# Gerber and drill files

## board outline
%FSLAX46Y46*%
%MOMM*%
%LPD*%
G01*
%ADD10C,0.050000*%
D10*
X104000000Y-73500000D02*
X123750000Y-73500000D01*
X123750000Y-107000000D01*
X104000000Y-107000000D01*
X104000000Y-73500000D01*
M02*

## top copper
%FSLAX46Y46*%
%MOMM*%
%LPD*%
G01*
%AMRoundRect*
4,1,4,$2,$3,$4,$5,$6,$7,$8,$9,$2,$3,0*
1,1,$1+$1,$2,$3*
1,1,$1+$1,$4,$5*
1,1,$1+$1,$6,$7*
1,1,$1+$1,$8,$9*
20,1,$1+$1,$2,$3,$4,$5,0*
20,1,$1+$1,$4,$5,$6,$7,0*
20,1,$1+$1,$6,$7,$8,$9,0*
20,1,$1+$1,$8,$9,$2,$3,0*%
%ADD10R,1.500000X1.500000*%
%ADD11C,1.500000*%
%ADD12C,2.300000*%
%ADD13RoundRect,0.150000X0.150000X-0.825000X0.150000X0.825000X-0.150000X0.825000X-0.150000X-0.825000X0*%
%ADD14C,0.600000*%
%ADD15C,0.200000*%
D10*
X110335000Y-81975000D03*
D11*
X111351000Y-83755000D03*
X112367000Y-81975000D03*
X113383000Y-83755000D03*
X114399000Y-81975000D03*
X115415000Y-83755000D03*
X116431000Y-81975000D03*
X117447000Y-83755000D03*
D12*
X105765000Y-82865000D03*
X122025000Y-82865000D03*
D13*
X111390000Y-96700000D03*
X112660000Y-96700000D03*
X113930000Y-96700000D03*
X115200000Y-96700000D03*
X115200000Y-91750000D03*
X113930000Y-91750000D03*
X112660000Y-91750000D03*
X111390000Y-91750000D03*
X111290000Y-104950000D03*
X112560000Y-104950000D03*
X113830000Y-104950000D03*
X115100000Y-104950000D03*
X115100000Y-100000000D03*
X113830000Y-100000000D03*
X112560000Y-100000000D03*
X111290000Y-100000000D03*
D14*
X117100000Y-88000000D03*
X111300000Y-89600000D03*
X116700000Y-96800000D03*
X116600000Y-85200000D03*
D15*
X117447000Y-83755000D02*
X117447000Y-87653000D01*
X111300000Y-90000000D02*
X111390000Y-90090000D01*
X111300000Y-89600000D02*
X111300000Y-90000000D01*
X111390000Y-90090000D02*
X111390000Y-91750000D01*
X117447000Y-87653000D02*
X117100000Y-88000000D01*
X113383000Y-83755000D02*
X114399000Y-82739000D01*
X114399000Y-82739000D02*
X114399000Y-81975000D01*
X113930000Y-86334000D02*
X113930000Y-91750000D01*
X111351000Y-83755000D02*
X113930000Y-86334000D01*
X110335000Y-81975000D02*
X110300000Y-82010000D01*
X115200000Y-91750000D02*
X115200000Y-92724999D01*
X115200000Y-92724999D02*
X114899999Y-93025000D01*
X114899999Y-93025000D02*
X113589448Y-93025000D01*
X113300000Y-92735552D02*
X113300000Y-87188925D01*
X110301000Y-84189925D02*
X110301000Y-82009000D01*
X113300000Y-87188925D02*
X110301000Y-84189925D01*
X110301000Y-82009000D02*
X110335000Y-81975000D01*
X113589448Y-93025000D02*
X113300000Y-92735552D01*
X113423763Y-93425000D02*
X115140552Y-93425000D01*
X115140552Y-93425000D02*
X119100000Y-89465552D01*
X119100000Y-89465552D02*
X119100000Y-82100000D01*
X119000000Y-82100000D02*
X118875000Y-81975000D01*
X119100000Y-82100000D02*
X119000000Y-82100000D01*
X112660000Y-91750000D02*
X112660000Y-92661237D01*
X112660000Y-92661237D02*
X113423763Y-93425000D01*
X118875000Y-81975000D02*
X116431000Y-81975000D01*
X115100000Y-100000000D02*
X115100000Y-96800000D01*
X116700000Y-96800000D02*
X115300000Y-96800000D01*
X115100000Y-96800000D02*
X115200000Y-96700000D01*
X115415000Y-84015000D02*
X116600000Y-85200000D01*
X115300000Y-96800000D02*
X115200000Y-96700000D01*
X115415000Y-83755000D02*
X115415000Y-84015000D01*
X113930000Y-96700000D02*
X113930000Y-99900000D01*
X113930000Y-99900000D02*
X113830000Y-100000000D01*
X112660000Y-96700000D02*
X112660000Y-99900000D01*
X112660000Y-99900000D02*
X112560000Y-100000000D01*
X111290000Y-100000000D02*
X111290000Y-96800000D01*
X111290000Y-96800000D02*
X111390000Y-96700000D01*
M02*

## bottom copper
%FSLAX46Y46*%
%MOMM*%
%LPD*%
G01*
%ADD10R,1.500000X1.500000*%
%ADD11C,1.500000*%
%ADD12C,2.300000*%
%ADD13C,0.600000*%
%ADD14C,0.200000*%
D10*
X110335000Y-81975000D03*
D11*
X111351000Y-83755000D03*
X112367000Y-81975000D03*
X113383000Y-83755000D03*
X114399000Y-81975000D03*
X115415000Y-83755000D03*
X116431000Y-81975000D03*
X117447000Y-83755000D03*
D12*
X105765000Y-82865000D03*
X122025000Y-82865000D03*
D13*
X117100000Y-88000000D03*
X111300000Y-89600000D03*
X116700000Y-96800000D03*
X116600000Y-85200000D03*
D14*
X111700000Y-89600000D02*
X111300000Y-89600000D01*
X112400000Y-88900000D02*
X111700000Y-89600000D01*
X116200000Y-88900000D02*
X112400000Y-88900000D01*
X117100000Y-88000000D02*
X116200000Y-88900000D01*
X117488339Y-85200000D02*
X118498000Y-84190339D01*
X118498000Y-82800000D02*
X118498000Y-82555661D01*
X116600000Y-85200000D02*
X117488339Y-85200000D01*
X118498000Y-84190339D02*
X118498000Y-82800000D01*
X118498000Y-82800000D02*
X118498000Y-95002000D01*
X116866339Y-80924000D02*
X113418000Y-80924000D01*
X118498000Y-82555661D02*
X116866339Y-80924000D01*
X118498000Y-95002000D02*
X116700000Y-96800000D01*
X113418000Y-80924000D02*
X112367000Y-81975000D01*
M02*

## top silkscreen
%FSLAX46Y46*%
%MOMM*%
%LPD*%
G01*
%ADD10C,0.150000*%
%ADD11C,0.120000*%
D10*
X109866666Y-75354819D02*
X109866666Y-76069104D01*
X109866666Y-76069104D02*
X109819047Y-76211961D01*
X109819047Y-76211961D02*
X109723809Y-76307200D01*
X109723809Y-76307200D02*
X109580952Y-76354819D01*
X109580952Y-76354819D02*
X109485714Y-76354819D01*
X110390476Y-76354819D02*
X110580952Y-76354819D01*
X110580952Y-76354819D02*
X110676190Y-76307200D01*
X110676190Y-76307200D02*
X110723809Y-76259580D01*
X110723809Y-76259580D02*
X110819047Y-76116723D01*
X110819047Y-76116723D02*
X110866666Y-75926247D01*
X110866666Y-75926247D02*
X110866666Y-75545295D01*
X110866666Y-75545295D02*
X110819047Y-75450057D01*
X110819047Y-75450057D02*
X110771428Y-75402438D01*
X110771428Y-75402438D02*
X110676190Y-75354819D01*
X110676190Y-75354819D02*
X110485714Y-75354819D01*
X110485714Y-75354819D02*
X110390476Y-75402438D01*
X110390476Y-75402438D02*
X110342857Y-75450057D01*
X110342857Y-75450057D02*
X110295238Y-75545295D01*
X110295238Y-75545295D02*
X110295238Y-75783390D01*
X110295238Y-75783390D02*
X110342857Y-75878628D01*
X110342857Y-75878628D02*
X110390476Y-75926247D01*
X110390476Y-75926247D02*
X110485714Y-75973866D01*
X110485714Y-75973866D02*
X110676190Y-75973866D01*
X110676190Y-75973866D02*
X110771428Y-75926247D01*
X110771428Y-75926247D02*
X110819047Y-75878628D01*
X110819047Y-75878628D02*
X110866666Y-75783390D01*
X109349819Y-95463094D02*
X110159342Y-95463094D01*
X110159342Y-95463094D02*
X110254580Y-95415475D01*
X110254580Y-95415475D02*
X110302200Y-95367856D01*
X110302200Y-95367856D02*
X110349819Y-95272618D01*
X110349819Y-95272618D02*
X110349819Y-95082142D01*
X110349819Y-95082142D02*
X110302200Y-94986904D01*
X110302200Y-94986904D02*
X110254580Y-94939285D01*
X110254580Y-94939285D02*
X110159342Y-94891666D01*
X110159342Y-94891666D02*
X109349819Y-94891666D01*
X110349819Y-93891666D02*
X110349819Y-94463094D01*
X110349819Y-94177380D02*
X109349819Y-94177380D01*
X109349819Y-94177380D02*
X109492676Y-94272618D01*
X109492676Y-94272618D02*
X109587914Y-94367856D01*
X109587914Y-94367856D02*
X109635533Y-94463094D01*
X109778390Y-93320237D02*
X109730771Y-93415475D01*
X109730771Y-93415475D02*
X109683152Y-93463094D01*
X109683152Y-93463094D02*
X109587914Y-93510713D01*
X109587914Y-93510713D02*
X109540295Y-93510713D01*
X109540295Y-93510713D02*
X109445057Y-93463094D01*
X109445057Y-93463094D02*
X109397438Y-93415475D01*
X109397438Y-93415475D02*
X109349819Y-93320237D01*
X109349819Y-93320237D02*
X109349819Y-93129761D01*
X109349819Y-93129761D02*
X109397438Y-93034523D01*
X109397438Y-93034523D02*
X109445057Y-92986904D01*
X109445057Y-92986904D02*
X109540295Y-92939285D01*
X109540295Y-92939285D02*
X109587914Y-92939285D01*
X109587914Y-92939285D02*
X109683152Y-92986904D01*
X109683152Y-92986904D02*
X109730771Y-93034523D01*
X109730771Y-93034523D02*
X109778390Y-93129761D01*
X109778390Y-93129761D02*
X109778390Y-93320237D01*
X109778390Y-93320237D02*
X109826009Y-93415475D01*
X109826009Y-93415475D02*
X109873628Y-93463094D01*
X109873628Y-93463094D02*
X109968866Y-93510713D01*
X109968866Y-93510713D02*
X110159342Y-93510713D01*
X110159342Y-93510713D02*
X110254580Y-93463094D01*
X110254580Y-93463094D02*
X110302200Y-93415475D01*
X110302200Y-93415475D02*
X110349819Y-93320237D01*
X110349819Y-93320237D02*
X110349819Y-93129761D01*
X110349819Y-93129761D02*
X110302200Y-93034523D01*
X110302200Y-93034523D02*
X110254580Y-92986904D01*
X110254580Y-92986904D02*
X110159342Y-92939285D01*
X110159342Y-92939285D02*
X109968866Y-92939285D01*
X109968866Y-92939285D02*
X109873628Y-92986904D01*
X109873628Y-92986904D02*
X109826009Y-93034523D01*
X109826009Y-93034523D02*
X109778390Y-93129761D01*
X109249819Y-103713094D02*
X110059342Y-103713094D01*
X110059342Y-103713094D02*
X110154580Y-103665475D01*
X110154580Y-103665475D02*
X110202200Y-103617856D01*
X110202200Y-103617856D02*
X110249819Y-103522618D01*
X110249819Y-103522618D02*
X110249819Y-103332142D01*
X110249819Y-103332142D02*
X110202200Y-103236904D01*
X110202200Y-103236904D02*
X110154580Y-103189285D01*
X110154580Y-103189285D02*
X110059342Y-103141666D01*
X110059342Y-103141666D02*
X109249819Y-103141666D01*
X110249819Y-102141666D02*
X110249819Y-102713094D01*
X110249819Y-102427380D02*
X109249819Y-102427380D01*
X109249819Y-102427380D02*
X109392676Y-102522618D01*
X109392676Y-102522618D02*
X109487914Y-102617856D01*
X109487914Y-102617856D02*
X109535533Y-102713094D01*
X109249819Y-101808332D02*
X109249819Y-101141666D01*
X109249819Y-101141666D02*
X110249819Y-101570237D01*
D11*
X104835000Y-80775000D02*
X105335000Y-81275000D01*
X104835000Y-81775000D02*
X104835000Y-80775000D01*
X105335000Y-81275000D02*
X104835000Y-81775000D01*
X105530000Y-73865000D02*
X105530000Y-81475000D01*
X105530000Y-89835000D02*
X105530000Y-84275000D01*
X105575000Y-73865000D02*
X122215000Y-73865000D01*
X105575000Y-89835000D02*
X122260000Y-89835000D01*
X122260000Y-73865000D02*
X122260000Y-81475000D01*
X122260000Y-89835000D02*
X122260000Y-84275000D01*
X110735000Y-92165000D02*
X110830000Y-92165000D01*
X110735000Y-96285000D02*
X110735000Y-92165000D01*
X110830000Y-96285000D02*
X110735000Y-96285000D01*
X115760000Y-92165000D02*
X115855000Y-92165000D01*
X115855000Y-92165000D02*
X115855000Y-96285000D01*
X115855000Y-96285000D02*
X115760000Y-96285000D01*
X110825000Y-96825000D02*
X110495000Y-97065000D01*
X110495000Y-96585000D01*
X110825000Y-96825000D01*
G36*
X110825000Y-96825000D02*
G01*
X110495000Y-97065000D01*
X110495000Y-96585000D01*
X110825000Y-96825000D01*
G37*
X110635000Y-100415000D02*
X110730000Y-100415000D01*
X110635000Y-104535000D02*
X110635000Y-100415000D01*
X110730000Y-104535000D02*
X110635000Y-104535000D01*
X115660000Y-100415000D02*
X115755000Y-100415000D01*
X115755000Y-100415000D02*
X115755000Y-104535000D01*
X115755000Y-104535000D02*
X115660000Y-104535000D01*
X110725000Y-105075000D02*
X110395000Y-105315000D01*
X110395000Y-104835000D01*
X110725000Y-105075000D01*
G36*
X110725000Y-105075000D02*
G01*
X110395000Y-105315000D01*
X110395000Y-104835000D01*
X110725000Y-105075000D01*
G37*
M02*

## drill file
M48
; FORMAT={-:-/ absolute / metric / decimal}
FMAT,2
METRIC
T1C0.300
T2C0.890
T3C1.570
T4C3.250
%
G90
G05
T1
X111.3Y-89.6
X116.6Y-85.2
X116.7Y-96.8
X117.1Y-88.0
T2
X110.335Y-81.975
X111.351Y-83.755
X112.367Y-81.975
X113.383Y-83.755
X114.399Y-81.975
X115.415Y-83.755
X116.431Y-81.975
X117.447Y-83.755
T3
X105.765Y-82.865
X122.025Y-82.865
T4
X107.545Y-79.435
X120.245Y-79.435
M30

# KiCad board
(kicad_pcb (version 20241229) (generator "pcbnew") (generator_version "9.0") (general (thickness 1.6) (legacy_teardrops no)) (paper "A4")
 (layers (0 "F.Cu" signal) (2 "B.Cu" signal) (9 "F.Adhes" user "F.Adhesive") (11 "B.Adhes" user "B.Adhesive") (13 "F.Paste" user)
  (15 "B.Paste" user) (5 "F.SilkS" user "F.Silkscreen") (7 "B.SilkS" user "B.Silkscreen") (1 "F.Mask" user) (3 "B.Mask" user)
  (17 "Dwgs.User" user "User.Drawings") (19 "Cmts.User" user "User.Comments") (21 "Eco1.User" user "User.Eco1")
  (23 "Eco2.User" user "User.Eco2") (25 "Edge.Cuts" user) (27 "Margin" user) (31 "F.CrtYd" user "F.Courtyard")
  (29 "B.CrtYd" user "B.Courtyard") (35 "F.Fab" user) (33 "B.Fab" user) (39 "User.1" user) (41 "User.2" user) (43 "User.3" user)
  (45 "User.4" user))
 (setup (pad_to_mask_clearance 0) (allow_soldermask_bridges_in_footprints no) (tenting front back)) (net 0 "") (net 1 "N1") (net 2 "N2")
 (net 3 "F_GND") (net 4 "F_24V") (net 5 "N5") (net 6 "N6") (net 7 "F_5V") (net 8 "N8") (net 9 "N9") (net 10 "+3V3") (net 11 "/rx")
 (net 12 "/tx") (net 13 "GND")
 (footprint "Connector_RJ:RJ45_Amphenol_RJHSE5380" (layer "F.Cu") (at 110.335 81.975)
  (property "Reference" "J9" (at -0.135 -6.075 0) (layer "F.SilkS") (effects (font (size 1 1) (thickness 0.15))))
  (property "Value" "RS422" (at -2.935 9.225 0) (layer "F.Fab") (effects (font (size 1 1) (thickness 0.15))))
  (fp_line (start -5.5 -1.2) (end -5 -0.7) (stroke (width 0.12) (type solid)) (layer "F.SilkS"))
  (fp_line (start -5.5 -0.2) (end -5.5 -1.2) (stroke (width 0.12) (type solid)) (layer "F.SilkS"))
  (fp_line (start -5 -0.7) (end -5.5 -0.2) (stroke (width 0.12) (type solid)) (layer "F.SilkS"))
  (fp_line (start -4.805 -8.11) (end -4.805 -0.5) (stroke (width 0.12) (type solid)) (layer "F.SilkS"))
  (fp_line (start -4.805 7.86) (end -4.805 2.3) (stroke (width 0.12) (type solid)) (layer "F.SilkS"))
  (fp_line (start -4.76 -8.11) (end 11.88 -8.11) (stroke (width 0.12) (type solid)) (layer "F.SilkS"))
  (fp_line (start -4.76 7.86) (end 11.925 7.86) (stroke (width 0.12) (type solid)) (layer "F.SilkS"))
  (fp_line (start 11.925 -8.11) (end 11.925 -0.5) (stroke (width 0.12) (type solid)) (layer "F.SilkS"))
  (fp_line (start 11.925 7.86) (end 11.925 2.3) (stroke (width 0.12) (type solid)) (layer "F.SilkS"))
  (pad "" np_thru_hole circle (at -2.79 -2.54) (size 3.25 3.25) (drill 3.25) (layers "*.Cu" "*.Mask"))
  (pad "" np_thru_hole circle (at 9.91 -2.54) (size 3.25 3.25) (drill 3.25) (layers "*.Cu" "*.Mask"))
  (pad "1" thru_hole rect (at 0 0) (size 1.5 1.5) (drill 0.89) (layers "*.Cu" "*.Mask") (remove_unused_layers no) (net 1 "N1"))
  (pad "2" thru_hole circle (at 1.016 1.78) (size 1.5 1.5) (drill 0.89) (layers "*.Cu" "*.Mask") (remove_unused_layers no) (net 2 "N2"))
  (pad "3" thru_hole circle (at 2.032 0) (size 1.5 1.5) (drill 0.89) (layers "*.Cu" "*.Mask") (remove_unused_layers no) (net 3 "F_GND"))
  (pad "4" thru_hole circle (at 3.048 1.78) (size 1.5 1.5) (drill 0.89) (layers "*.Cu" "*.Mask") (remove_unused_layers no) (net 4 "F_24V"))
  (pad "5" thru_hole circle (at 4.064 0) (size 1.5 1.5) (drill 0.89) (layers "*.Cu" "*.Mask") (remove_unused_layers no) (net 4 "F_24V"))
  (pad "6" thru_hole circle (at 5.08 1.78) (size 1.5 1.5) (drill 0.89) (layers "*.Cu" "*.Mask") (remove_unused_layers no) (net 3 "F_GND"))
  (pad "7" thru_hole circle (at 6.096 0) (size 1.5 1.5) (drill 0.89) (layers "*.Cu" "*.Mask") (remove_unused_layers no) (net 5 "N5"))
  (pad "8" thru_hole circle (at 7.112 1.78) (size 1.5 1.5) (drill 0.89) (layers "*.Cu" "*.Mask") (remove_unused_layers no) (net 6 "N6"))
  (pad "SH" thru_hole circle (at -4.57 0.89) (size 2.3 2.3) (drill 1.57) (layers "*.Cu" "*.Mask") (remove_unused_layers no))
  (pad "SH" thru_hole circle (at 11.69 0.89) (size 2.3 2.3) (drill 1.57) (layers "*.Cu" "*.Mask") (remove_unused_layers no)))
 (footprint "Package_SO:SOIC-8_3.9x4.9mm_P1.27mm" (layer "F.Cu") (at 113.295 94.225 90)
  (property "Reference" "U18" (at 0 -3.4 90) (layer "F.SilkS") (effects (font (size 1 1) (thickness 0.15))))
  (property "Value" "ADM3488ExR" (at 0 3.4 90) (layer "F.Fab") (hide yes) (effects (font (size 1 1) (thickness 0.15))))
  (fp_line (start 2.06 -2.56) (end 2.06 -2.465) (stroke (width 0.12) (type solid)) (layer "F.SilkS"))
  (fp_line (start -2.06 -2.56) (end 2.06 -2.56) (stroke (width 0.12) (type solid)) (layer "F.SilkS"))
  (fp_line (start -2.06 -2.465) (end -2.06 -2.56) (stroke (width 0.12) (type solid)) (layer "F.SilkS"))
  (fp_line (start 2.06 2.465) (end 2.06 2.56) (stroke (width 0.12) (type solid)) (layer "F.SilkS"))
  (fp_line (start 2.06 2.56) (end -2.06 2.56) (stroke (width 0.12) (type solid)) (layer "F.SilkS"))
  (fp_line (start -2.06 2.56) (end -2.06 2.465) (stroke (width 0.12) (type solid)) (layer "F.SilkS"))
  (fp_poly (pts (xy -2.6 -2.47) (xy -2.84 -2.8) (xy -2.36 -2.8)) (stroke (width 0.12) (type solid)) (fill yes) (layer "F.SilkS"))
  (pad "1" smd roundrect (at -2.475 -1.905 90) (size 1.95 0.6) (layers "F.Cu" "F.Mask" "F.Paste") (roundrect_rratio 0.25) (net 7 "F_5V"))
  (pad "2" smd roundrect (at -2.475 -0.635 90) (size 1.95 0.6) (layers "F.Cu" "F.Mask" "F.Paste") (roundrect_rratio 0.25) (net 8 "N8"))
  (pad "3" smd roundrect (at -2.475 0.635 90) (size 1.95 0.6) (layers "F.Cu" "F.Mask" "F.Paste") (roundrect_rratio 0.25) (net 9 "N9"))
  (pad "4" smd roundrect (at -2.475 1.905 90) (size 1.95 0.6) (layers "F.Cu" "F.Mask" "F.Paste") (roundrect_rratio 0.25) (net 3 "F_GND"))
  (pad "5" smd roundrect (at 2.475 1.905 90) (size 1.95 0.6) (layers "F.Cu" "F.Mask" "F.Paste") (roundrect_rratio 0.25) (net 1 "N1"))
  (pad "6" smd roundrect (at 2.475 0.635 90) (size 1.95 0.6) (layers "F.Cu" "F.Mask" "F.Paste") (roundrect_rratio 0.25) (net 2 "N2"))
  (pad "7" smd roundrect (at 2.475 -0.635 90) (size 1.95 0.6) (layers "F.Cu" "F.Mask" "F.Paste") (roundrect_rratio 0.25) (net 5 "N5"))
  (pad "8" smd roundrect (at 2.475 -1.905 90) (size 1.95 0.6) (layers "F.Cu" "F.Mask" "F.Paste") (roundrect_rratio 0.25) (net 6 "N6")))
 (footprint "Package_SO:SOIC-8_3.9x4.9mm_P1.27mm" (layer "F.Cu") (at 113.195 102.475 90)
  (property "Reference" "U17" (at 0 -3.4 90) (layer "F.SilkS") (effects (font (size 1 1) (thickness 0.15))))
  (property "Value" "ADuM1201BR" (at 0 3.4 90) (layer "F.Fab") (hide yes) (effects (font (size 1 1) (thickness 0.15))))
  (fp_line (start 2.06 -2.56) (end 2.06 -2.465) (stroke (width 0.12) (type solid)) (layer "F.SilkS"))
  (fp_line (start -2.06 -2.56) (end 2.06 -2.56) (stroke (width 0.12) (type solid)) (layer "F.SilkS"))
  (fp_line (start -2.06 -2.465) (end -2.06 -2.56) (stroke (width 0.12) (type solid)) (layer "F.SilkS"))
  (fp_line (start 2.06 2.465) (end 2.06 2.56) (stroke (width 0.12) (type solid)) (layer "F.SilkS"))
  (fp_line (start 2.06 2.56) (end -2.06 2.56) (stroke (width 0.12) (type solid)) (layer "F.SilkS"))
  (fp_line (start -2.06 2.56) (end -2.06 2.465) (stroke (width 0.12) (type solid)) (layer "F.SilkS"))
  (fp_poly (pts (xy -2.6 -2.47) (xy -2.84 -2.8) (xy -2.36 -2.8)) (stroke (width 0.12) (type solid)) (fill yes) (layer "F.SilkS"))
  (pad "1" smd roundrect (at -2.475 -1.905 90) (size 1.95 0.6) (layers "F.Cu" "F.Mask" "F.Paste") (roundrect_rratio 0.25) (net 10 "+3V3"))
  (pad "2" smd roundrect (at -2.475 -0.635 90) (size 1.95 0.6) (layers "F.Cu" "F.Mask" "F.Paste") (roundrect_rratio 0.25) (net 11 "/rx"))
  (pad "3" smd roundrect (at -2.475 0.635 90) (size 1.95 0.6) (layers "F.Cu" "F.Mask" "F.Paste") (roundrect_rratio 0.25) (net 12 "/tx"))
  (pad "4" smd roundrect (at -2.475 1.905 90) (size 1.95 0.6) (layers "F.Cu" "F.Mask" "F.Paste") (roundrect_rratio 0.25) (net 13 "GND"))
  (pad "5" smd roundrect (at 2.475 1.905 90) (size 1.95 0.6) (layers "F.Cu" "F.Mask" "F.Paste") (roundrect_rratio 0.25) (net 3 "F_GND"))
  (pad "6" smd roundrect (at 2.475 0.635 90) (size 1.95 0.6) (layers "F.Cu" "F.Mask" "F.Paste") (roundrect_rratio 0.25) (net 9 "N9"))
  (pad "7" smd roundrect (at 2.475 -0.635 90) (size 1.95 0.6) (layers "F.Cu" "F.Mask" "F.Paste") (roundrect_rratio 0.25) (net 8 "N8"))
  (pad "8" smd roundrect (at 2.475 -1.905 90) (size 1.95 0.6) (layers "F.Cu" "F.Mask" "F.Paste") (roundrect_rratio 0.25) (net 7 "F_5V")))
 (gr_rect (start 104 73.5) (end 123.75 107) (stroke (width 0.05) (type default)) (fill no) (layer "Edge.Cuts"))
 (segment (start 117.447 83.755) (end 117.447 87.653) (width 0.2) (layer "F.Cu") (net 6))
 (segment (start 111.3 90) (end 111.39 90.09) (width 0.2) (layer "F.Cu") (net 6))
 (segment (start 111.3 89.6) (end 111.3 90) (width 0.2) (layer "F.Cu") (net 6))
 (segment (start 111.39 90.09) (end 111.39 91.75) (width 0.2) (layer "F.Cu") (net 6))
 (segment (start 117.447 87.653) (end 117.1 88) (width 0.2) (layer "F.Cu") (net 6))
 (via (at 117.1 88) (size 0.6) (drill 0.3) (layers "F.Cu" "B.Cu") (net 6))
 (via (at 111.3 89.6) (size 0.6) (drill 0.3) (layers "F.Cu" "B.Cu") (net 6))
 (segment (start 111.7 89.6) (end 111.3 89.6) (width 0.2) (layer "B.Cu") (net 6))
 (segment (start 112.4 88.9) (end 111.7 89.6) (width 0.2) (layer "B.Cu") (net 6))
 (segment (start 116.2 88.9) (end 112.4 88.9) (width 0.2) (layer "B.Cu") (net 6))
 (segment (start 117.1 88) (end 116.2 88.9) (width 0.2) (layer "B.Cu") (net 6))
 (segment (start 113.383 83.755) (end 114.399 82.739) (width 0.2) (layer "F.Cu") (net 4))
 (segment (start 114.399 82.739) (end 114.399 81.975) (width 0.2) (layer "F.Cu") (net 4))
 (segment (start 113.93 86.334) (end 113.93 91.75) (width 0.2) (layer "F.Cu") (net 2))
 (segment (start 111.351 83.755) (end 113.93 86.334) (width 0.2) (layer "F.Cu") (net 2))
 (segment (start 110.335 81.975) (end 110.3 82.01) (width 0.2) (layer "F.Cu") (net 1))
 (segment (start 115.2 91.75) (end 115.2 92.724999) (width 0.2) (layer "F.Cu") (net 1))
 (segment (start 115.2 92.724999) (end 114.899999 93.025) (width 0.2) (layer "F.Cu") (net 1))
 (segment (start 114.899999 93.025) (end 113.589448 93.025) (width 0.2) (layer "F.Cu") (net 1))
 (segment (start 113.3 92.735552) (end 113.3 87.188925) (width 0.2) (layer "F.Cu") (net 1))
 (segment (start 110.301 84.189925) (end 110.301 82.009) (width 0.2) (layer "F.Cu") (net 1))
 (segment (start 113.3 87.188925) (end 110.301 84.189925) (width 0.2) (layer "F.Cu") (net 1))
 (segment (start 110.301 82.009) (end 110.335 81.975) (width 0.2) (layer "F.Cu") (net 1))
 (segment (start 113.589448 93.025) (end 113.3 92.735552) (width 0.2) (layer "F.Cu") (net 1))
 (segment (start 113.423763 93.425) (end 115.140552 93.425) (width 0.2) (layer "F.Cu") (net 5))
 (segment (start 115.140552 93.425) (end 119.1 89.465552) (width 0.2) (layer "F.Cu") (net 5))
 (segment (start 119.1 89.465552) (end 119.1 82.1) (width 0.2) (layer "F.Cu") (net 5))
 (segment (start 119 82.1) (end 118.875 81.975) (width 0.2) (layer "F.Cu") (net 5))
 (segment (start 119.1 82.1) (end 119 82.1) (width 0.2) (layer "F.Cu") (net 5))
 (segment (start 112.66 91.75) (end 112.66 92.661237) (width 0.2) (layer "F.Cu") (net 5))
 (segment (start 112.66 92.661237) (end 113.423763 93.425) (width 0.2) (layer "F.Cu") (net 5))
 (segment (start 118.875 81.975) (end 116.431 81.975) (width 0.2) (layer "F.Cu") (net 5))
 (segment (start 115.1 100) (end 115.1 96.8) (width 0.2) (layer "F.Cu") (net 3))
 (segment (start 116.7 96.8) (end 115.3 96.8) (width 0.2) (layer "F.Cu") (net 3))
 (segment (start 115.1 96.8) (end 115.2 96.7) (width 0.2) (layer "F.Cu") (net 3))
 (segment (start 115.415 84.015) (end 116.6 85.2) (width 0.2) (layer "F.Cu") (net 3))
 (segment (start 115.3 96.8) (end 115.2 96.7) (width 0.2) (layer "F.Cu") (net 3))
 (segment (start 115.415 83.755) (end 115.415 84.015) (width 0.2) (layer "F.Cu") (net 3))
 (via (at 116.7 96.8) (size 0.6) (drill 0.3) (layers "F.Cu" "B.Cu") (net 3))
 (via (at 116.6 85.2) (size 0.6) (drill 0.3) (layers "F.Cu" "B.Cu") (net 3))
 (segment (start 117.488339 85.2) (end 118.498 84.190339) (width 0.2) (layer "B.Cu") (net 3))
 (segment (start 118.498 82.8) (end 118.498 82.555661) (width 0.2) (layer "B.Cu") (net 3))
 (segment (start 116.6 85.2) (end 117.488339 85.2) (width 0.2) (layer "B.Cu") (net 3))
 (segment (start 118.498 84.190339) (end 118.498 82.8) (width 0.2) (layer "B.Cu") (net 3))
 (segment (start 118.498 82.8) (end 118.498 95.002) (width 0.2) (layer "B.Cu") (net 3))
 (segment (start 116.866339 80.924) (end 113.418 80.924) (width 0.2) (layer "B.Cu") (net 3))
 (segment (start 118.498 82.555661) (end 116.866339 80.924) (width 0.2) (layer "B.Cu") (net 3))
 (segment (start 118.498 95.002) (end 116.7 96.8) (width 0.2) (layer "B.Cu") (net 3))
 (segment (start 113.418 80.924) (end 112.367 81.975) (width 0.2) (layer "B.Cu") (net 3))
 (segment (start 113.93 96.7) (end 113.93 99.9) (width 0.2) (layer "F.Cu") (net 9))
 (segment (start 113.93 99.9) (end 113.83 100) (width 0.2) (layer "F.Cu") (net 9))
 (segment (start 112.66 96.7) (end 112.66 99.9) (width 0.2) (layer "F.Cu") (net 8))
 (segment (start 112.66 99.9) (end 112.56 100) (width 0.2) (layer "F.Cu") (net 8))
 (segment (start 111.29 100) (end 111.29 96.8) (width 0.2) (layer "F.Cu") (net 7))
 (segment (start 111.29 96.8) (end 111.39 96.7) (width 0.2) (layer "F.Cu") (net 7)))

